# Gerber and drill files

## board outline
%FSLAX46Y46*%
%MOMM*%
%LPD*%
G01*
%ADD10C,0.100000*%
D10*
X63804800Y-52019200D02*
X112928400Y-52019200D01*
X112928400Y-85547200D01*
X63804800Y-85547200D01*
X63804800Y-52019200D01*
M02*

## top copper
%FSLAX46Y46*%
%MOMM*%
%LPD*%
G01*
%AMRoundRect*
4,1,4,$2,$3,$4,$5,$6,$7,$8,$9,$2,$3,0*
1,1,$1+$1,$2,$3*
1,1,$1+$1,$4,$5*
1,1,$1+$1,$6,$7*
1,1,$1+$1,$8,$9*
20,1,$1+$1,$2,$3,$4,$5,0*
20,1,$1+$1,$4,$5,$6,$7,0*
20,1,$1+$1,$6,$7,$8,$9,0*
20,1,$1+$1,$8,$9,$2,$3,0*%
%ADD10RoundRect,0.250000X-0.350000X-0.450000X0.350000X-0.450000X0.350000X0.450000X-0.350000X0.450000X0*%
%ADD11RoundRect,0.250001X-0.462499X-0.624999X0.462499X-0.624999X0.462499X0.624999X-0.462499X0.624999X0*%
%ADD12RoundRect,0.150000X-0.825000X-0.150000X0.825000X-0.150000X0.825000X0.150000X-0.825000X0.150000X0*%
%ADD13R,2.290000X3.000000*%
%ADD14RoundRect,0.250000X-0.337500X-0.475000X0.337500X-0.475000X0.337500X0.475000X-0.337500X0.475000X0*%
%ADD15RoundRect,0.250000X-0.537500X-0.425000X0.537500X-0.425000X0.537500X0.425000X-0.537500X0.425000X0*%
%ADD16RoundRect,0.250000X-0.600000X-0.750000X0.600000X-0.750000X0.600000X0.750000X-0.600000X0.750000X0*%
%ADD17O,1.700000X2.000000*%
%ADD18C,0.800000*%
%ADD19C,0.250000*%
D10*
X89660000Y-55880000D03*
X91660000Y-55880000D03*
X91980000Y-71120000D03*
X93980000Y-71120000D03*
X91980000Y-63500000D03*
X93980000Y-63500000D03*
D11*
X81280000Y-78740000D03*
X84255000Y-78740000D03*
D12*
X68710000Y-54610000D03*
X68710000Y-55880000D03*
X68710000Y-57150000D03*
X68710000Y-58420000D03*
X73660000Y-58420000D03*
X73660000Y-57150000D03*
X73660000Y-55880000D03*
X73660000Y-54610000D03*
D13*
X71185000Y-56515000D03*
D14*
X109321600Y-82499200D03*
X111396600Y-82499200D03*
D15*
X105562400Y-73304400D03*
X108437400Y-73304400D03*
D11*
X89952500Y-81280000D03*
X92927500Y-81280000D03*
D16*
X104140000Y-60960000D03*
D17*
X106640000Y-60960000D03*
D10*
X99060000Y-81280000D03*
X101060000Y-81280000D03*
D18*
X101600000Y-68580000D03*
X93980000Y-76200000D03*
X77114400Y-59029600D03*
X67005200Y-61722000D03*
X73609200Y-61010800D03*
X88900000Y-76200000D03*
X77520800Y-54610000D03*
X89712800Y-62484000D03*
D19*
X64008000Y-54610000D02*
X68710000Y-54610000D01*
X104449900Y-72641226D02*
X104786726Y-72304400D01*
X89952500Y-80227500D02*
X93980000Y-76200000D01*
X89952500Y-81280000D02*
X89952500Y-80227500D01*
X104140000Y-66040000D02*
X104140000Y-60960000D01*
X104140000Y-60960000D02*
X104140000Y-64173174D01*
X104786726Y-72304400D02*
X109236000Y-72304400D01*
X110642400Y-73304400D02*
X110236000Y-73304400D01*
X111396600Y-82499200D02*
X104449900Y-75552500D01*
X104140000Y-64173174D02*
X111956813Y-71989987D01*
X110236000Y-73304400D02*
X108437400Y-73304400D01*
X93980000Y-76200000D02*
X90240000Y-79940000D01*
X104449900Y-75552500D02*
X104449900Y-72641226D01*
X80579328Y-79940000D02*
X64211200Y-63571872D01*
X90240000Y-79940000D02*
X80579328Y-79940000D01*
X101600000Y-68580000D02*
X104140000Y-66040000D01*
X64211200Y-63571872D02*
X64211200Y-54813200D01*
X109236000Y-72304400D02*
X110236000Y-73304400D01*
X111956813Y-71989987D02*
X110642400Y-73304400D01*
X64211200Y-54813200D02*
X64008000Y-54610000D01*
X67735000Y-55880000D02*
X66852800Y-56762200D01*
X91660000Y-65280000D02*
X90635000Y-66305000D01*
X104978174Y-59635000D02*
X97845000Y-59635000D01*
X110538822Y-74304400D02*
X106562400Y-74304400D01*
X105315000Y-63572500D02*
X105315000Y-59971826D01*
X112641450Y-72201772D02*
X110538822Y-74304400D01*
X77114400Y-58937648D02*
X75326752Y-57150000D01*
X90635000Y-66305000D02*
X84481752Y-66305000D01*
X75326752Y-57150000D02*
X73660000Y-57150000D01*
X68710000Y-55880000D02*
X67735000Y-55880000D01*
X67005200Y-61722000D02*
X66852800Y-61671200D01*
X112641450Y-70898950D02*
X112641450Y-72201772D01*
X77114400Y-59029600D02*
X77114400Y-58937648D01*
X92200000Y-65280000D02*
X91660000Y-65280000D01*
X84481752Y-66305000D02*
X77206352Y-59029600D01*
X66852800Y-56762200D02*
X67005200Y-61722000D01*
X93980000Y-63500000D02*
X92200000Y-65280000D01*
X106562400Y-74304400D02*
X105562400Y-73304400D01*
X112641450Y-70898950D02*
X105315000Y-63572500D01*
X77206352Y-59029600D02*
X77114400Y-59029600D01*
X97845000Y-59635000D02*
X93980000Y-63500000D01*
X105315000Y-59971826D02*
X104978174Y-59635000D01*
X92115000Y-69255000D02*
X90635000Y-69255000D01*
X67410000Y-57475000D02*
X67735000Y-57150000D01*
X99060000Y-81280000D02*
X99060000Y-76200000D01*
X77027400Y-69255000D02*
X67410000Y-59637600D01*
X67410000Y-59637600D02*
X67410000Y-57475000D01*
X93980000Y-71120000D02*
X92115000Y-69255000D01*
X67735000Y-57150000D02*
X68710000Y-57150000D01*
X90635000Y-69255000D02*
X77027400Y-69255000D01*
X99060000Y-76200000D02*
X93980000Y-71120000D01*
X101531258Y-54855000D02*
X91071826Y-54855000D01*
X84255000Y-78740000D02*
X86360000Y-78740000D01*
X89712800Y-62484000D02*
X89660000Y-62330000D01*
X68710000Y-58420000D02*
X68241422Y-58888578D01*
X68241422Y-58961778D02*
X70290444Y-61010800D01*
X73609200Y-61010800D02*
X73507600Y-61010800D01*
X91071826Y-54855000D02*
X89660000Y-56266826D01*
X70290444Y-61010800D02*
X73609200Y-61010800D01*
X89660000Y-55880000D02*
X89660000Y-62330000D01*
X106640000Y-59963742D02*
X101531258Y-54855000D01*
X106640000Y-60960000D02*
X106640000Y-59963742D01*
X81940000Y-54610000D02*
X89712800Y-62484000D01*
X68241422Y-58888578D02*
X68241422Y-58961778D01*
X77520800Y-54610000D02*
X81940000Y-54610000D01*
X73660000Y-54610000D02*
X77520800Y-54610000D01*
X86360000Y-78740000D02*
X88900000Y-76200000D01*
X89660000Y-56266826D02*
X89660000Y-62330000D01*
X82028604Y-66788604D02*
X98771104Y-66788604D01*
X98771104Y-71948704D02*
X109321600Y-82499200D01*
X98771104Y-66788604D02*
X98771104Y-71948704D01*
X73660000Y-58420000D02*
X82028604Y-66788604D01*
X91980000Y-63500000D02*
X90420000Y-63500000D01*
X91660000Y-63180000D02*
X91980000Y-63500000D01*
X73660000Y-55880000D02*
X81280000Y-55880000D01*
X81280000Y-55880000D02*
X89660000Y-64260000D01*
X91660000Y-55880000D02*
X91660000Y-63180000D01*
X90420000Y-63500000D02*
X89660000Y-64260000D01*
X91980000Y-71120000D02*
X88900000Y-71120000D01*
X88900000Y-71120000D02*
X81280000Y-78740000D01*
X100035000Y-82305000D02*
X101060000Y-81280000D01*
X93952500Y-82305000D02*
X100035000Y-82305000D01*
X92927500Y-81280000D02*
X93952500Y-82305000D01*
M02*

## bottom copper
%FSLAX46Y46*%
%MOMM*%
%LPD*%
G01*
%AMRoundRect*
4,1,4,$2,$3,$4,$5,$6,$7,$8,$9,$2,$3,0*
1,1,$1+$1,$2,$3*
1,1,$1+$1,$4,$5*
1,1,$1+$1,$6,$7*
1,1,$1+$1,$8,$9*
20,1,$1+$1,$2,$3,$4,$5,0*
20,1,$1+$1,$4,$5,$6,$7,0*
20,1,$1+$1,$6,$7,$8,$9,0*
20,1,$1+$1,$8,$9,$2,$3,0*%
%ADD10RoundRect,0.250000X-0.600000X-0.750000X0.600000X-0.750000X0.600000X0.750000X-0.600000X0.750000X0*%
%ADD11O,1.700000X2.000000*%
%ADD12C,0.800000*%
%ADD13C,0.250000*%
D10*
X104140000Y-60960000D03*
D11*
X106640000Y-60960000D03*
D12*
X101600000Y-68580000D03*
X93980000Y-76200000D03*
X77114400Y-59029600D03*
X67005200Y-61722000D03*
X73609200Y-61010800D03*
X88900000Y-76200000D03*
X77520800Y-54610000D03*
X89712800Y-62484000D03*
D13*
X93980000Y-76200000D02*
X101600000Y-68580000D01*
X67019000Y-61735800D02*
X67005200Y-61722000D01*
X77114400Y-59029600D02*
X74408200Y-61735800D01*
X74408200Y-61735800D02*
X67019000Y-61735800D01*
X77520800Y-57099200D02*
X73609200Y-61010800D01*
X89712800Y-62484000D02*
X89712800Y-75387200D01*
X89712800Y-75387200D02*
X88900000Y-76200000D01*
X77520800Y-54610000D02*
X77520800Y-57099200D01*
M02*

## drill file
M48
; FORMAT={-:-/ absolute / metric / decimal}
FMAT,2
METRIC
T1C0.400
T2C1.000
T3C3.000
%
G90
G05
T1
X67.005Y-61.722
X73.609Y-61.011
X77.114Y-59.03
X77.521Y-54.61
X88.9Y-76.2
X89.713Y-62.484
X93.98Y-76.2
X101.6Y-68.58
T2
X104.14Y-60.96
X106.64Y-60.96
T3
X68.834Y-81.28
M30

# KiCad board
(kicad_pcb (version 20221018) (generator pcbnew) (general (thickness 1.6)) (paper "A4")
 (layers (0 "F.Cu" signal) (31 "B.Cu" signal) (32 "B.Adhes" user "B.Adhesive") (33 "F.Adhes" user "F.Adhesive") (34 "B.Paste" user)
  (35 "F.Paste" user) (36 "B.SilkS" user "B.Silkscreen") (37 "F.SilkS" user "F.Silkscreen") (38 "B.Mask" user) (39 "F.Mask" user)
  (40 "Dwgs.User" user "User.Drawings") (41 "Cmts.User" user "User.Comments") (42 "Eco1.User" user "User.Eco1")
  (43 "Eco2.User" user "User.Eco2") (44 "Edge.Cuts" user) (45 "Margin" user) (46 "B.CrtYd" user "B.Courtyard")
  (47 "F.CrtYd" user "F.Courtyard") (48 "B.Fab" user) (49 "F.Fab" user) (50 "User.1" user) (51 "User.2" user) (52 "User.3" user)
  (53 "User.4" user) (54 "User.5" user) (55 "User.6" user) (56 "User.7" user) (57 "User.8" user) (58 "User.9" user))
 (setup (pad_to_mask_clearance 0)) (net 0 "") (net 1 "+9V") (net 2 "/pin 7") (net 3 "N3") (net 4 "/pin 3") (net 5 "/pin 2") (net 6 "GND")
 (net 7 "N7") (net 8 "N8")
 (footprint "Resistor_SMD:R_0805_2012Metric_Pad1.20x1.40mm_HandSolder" (layer "F.Cu") (at 90.66 55.88)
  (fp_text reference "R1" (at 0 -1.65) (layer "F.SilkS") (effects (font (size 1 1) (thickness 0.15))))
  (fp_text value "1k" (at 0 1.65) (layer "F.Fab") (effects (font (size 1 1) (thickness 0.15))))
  (pad "1" smd roundrect (at -1 0) (size 1.2 1.4) (layers "F.Cu" "F.Paste" "F.Mask") (roundrect_rratio 0.2083333333) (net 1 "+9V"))
  (pad "2" smd roundrect (at 1 0) (size 1.2 1.4) (layers "F.Cu" "F.Paste" "F.Mask") (roundrect_rratio 0.2083333333) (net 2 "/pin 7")))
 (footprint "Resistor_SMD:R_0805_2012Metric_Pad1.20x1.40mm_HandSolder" (layer "F.Cu") (at 92.98 71.12)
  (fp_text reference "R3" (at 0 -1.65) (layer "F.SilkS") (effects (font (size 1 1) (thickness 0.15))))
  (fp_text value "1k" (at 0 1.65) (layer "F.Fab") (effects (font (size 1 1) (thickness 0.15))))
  (pad "1" smd roundrect (at -1 0) (size 1.2 1.4) (layers "F.Cu" "F.Paste" "F.Mask") (roundrect_rratio 0.2083333333) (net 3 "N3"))
  (pad "2" smd roundrect (at 1 0) (size 1.2 1.4) (layers "F.Cu" "F.Paste" "F.Mask") (roundrect_rratio 0.2083333333) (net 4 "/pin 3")))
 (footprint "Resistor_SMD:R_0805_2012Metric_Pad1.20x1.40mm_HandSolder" (layer "F.Cu") (at 92.98 63.5)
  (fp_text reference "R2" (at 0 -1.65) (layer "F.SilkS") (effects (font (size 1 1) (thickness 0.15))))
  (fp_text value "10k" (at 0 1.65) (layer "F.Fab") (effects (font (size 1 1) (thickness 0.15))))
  (pad "1" smd roundrect (at -1 0) (size 1.2 1.4) (layers "F.Cu" "F.Paste" "F.Mask") (roundrect_rratio 0.2083333333) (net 2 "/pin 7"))
  (pad "2" smd roundrect (at 1 0) (size 1.2 1.4) (layers "F.Cu" "F.Paste" "F.Mask") (roundrect_rratio 0.2083333333) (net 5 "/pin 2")))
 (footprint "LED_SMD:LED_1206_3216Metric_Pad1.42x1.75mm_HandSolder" (layer "F.Cu") (at 82.7675 78.74)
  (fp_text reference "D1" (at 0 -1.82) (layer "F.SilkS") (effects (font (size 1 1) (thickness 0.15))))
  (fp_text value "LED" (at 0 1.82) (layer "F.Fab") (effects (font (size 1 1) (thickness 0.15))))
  (pad "1" smd roundrect (at -1.4875 0) (size 1.425 1.75) (layers "F.Cu" "F.Paste" "F.Mask") (roundrect_rratio 0.1754392982) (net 3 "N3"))
  (pad "2" smd roundrect (at 1.4875 0) (size 1.425 1.75) (layers "F.Cu" "F.Paste" "F.Mask") (roundrect_rratio 0.1754392982) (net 1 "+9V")))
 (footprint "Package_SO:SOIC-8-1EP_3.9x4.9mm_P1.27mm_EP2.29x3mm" (layer "F.Cu") (at 71.185 56.515)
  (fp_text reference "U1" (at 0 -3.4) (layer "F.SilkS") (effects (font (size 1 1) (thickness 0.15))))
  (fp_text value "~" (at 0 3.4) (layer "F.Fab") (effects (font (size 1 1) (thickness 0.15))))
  (pad "" smd roundrect (at -0.57 -0.75) (size 0.92 1.21) (layers "F.Paste") (roundrect_rratio 0.25))
  (pad "" smd roundrect (at -0.57 0.75) (size 0.92 1.21) (layers "F.Paste") (roundrect_rratio 0.25))
  (pad "" smd roundrect (at 0.57 -0.75) (size 0.92 1.21) (layers "F.Paste") (roundrect_rratio 0.25))
  (pad "" smd roundrect (at 0.57 0.75) (size 0.92 1.21) (layers "F.Paste") (roundrect_rratio 0.25))
  (pad "1" smd roundrect (at -2.475 -1.905) (size 1.95 0.6) (layers "F.Cu" "F.Paste" "F.Mask") (roundrect_rratio 0.25) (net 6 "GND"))
  (pad "2" smd roundrect (at -2.475 -0.635) (size 1.95 0.6) (layers "F.Cu" "F.Paste" "F.Mask") (roundrect_rratio 0.25) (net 5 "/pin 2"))
  (pad "3" smd roundrect (at -2.475 0.635) (size 1.95 0.6) (layers "F.Cu" "F.Paste" "F.Mask") (roundrect_rratio 0.25) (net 4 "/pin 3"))
  (pad "4" smd roundrect (at -2.475 1.905) (size 1.95 0.6) (layers "F.Cu" "F.Paste" "F.Mask") (roundrect_rratio 0.25) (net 1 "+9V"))
  (pad "5" smd roundrect (at 2.475 1.905) (size 1.95 0.6) (layers "F.Cu" "F.Paste" "F.Mask") (roundrect_rratio 0.25) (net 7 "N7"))
  (pad "6" smd roundrect (at 2.475 0.635) (size 1.95 0.6) (layers "F.Cu" "F.Paste" "F.Mask") (roundrect_rratio 0.25) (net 5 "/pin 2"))
  (pad "7" smd roundrect (at 2.475 -0.635) (size 1.95 0.6) (layers "F.Cu" "F.Paste" "F.Mask") (roundrect_rratio 0.25) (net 2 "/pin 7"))
  (pad "8" smd roundrect (at 2.475 -1.905) (size 1.95 0.6) (layers "F.Cu" "F.Paste" "F.Mask") (roundrect_rratio 0.25) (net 1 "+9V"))
  (pad "9" smd rect (at 0 0) (size 2.29 3) (layers "F.Cu" "F.Mask")))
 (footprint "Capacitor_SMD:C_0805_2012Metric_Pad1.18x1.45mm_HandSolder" (layer "F.Cu") (at 110.3591 82.4992)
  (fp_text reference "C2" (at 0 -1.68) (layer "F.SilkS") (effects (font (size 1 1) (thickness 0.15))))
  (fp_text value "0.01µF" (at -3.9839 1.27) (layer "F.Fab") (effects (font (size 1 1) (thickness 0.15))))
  (pad "1" smd roundrect (at -1.0375 0) (size 1.175 1.45) (layers "F.Cu" "F.Paste" "F.Mask") (roundrect_rratio 0.2127659574) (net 7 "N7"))
  (pad "2" smd roundrect (at 1.0375 0) (size 1.175 1.45) (layers "F.Cu" "F.Paste" "F.Mask") (roundrect_rratio 0.2127659574) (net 6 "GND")))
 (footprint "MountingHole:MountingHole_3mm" (layer "F.Cu") (at 68.834 81.28)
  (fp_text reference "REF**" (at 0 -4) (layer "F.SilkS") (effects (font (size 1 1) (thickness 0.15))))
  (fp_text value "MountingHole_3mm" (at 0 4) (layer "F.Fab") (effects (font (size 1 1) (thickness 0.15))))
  (pad "" np_thru_hole circle (at 0 0) (size 3 3) (drill 3) (layers "*.Cu" "*.Mask")))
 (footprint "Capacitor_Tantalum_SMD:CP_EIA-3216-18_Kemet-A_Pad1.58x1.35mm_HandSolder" (layer "F.Cu") (at 106.9999 73.3044)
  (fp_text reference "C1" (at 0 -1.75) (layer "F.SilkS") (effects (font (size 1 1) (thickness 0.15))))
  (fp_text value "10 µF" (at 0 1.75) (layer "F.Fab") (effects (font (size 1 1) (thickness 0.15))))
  (pad "1" smd roundrect (at -1.4375 0) (size 1.575 1.35) (layers "F.Cu" "F.Paste" "F.Mask") (roundrect_rratio 0.1851851852)
   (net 5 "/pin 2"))
  (pad "2" smd roundrect (at 1.4375 0) (size 1.575 1.35) (layers "F.Cu" "F.Paste" "F.Mask") (roundrect_rratio 0.1851851852) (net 6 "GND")))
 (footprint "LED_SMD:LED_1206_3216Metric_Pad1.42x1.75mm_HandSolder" (layer "F.Cu") (at 91.44 81.28)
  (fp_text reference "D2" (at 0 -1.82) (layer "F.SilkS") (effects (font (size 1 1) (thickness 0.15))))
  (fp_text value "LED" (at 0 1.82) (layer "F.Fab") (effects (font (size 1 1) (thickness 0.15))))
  (pad "1" smd roundrect (at -1.4875 0) (size 1.425 1.75) (layers "F.Cu" "F.Paste" "F.Mask") (roundrect_rratio 0.1754392982) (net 6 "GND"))
  (pad "2" smd roundrect (at 1.4875 0) (size 1.425 1.75) (layers "F.Cu" "F.Paste" "F.Mask") (roundrect_rratio 0.1754392982) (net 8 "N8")))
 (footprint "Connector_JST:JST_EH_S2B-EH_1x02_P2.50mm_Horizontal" (layer "F.Cu") (at 104.14 60.96)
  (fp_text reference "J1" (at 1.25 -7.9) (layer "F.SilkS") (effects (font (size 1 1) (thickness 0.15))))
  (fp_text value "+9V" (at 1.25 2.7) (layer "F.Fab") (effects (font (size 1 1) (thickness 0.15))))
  (pad "1" thru_hole roundrect (at 0 0) (size 1.7 2) (drill 1) (layers "*.Cu" "*.Mask") (roundrect_rratio 0.1470588235) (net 6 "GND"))
  (pad "2" thru_hole oval (at 2.5 0) (size 1.7 2) (drill 1) (layers "*.Cu" "*.Mask") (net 1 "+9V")))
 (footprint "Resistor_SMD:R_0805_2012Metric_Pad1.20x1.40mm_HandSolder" (layer "F.Cu") (at 100.06 81.28)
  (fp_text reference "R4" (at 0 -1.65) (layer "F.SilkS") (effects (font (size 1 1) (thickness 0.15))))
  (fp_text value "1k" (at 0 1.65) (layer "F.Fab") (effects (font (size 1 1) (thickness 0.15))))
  (pad "1" smd roundrect (at -1 0) (size 1.2 1.4) (layers "F.Cu" "F.Paste" "F.Mask") (roundrect_rratio 0.2083333333) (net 4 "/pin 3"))
  (pad "2" smd roundrect (at 1 0) (size 1.2 1.4) (layers "F.Cu" "F.Paste" "F.Mask") (roundrect_rratio 0.2083333333) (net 8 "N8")))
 (gr_rect (start 63.8048 52.0192) (end 112.9284 85.5472) (stroke (width 0.1) (type default)) (fill none) (layer "Edge.Cuts"))
 (segment (start 64.008 54.61) (end 68.71 54.61) (width 0.25) (layer "F.Cu") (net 6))
 (segment (start 104.4499 72.641226) (end 104.786726 72.3044) (width 0.25) (layer "F.Cu") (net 6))
 (segment (start 89.9525 80.2275) (end 93.98 76.2) (width 0.25) (layer "F.Cu") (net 6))
 (segment (start 89.9525 81.28) (end 89.9525 80.2275) (width 0.25) (layer "F.Cu") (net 6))
 (segment (start 104.14 66.04) (end 104.14 60.96) (width 0.25) (layer "F.Cu") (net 6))
 (segment (start 104.14 60.96) (end 104.14 64.173174) (width 0.25) (layer "F.Cu") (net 6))
 (segment (start 104.786726 72.3044) (end 109.236 72.3044) (width 0.25) (layer "F.Cu") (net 6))
 (segment (start 110.6424 73.3044) (end 110.236 73.3044) (width 0.25) (layer "F.Cu") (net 6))
 (segment (start 111.3966 82.4992) (end 104.4499 75.5525) (width 0.25) (layer "F.Cu") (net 6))
 (segment (start 104.14 64.173174) (end 111.956813 71.989987) (width 0.25) (layer "F.Cu") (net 6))
 (segment (start 110.236 73.3044) (end 108.4374 73.3044) (width 0.25) (layer "F.Cu") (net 6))
 (segment (start 93.98 76.2) (end 90.24 79.94) (width 0.25) (layer "F.Cu") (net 6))
 (segment (start 104.4499 75.5525) (end 104.4499 72.641226) (width 0.25) (layer "F.Cu") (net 6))
 (segment (start 80.579328 79.94) (end 64.2112 63.571872) (width 0.25) (layer "F.Cu") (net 6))
 (segment (start 90.24 79.94) (end 80.579328 79.94) (width 0.25) (layer "F.Cu") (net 6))
 (segment (start 101.6 68.58) (end 104.14 66.04) (width 0.25) (layer "F.Cu") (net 6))
 (segment (start 64.2112 63.571872) (end 64.2112 54.8132) (width 0.25) (layer "F.Cu") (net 6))
 (segment (start 109.236 72.3044) (end 110.236 73.3044) (width 0.25) (layer "F.Cu") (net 6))
 (segment (start 111.956813 71.989987) (end 110.6424 73.3044) (width 0.25) (layer "F.Cu") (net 6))
 (segment (start 64.2112 54.8132) (end 64.008 54.61) (width 0.25) (layer "F.Cu") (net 6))
 (via (at 101.6 68.58) (size 0.8) (drill 0.4) (layers "F.Cu" "B.Cu") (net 6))
 (via (at 93.98 76.2) (size 0.8) (drill 0.4) (layers "F.Cu" "B.Cu") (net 6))
 (segment (start 93.98 76.2) (end 101.6 68.58) (width 0.25) (layer "B.Cu") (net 6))
 (segment (start 67.735 55.88) (end 66.8528 56.7622) (width 0.25) (layer "F.Cu") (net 5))
 (segment (start 91.66 65.28) (end 90.635 66.305) (width 0.25) (layer "F.Cu") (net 5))
 (segment (start 104.978174 59.635) (end 97.845 59.635) (width 0.25) (layer "F.Cu") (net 5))
 (segment (start 110.538822 74.3044) (end 106.5624 74.3044) (width 0.25) (layer "F.Cu") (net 5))
 (segment (start 105.315 63.5725) (end 105.315 59.971826) (width 0.25) (layer "F.Cu") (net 5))
 (segment (start 112.64145 72.201772) (end 110.538822 74.3044) (width 0.25) (layer "F.Cu") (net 5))
 (segment (start 77.1144 58.937648) (end 75.326752 57.15) (width 0.25) (layer "F.Cu") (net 5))
 (segment (start 90.635 66.305) (end 84.481752 66.305) (width 0.25) (layer "F.Cu") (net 5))
 (segment (start 75.326752 57.15) (end 73.66 57.15) (width 0.25) (layer "F.Cu") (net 5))
 (segment (start 68.71 55.88) (end 67.735 55.88) (width 0.25) (layer "F.Cu") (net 5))
 (segment (start 67.0052 61.722) (end 66.8528 61.6712) (width 0.25) (layer "F.Cu") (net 5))
 (segment (start 112.64145 70.89895) (end 112.64145 72.201772) (width 0.25) (layer "F.Cu") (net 5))
 (segment (start 77.1144 59.0296) (end 77.1144 58.937648) (width 0.25) (layer "F.Cu") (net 5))
 (segment (start 92.2 65.28) (end 91.66 65.28) (width 0.25) (layer "F.Cu") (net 5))
 (segment (start 84.481752 66.305) (end 77.206352 59.0296) (width 0.25) (layer "F.Cu") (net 5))
 (segment (start 66.8528 56.7622) (end 67.0052 61.722) (width 0.25) (layer "F.Cu") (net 5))
 (segment (start 93.98 63.5) (end 92.2 65.28) (width 0.25) (layer "F.Cu") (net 5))
 (segment (start 106.5624 74.3044) (end 105.5624 73.3044) (width 0.25) (layer "F.Cu") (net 5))
 (segment (start 112.64145 70.89895) (end 105.315 63.5725) (width 0.25) (layer "F.Cu") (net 5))
 (segment (start 77.206352 59.0296) (end 77.1144 59.0296) (width 0.25) (layer "F.Cu") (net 5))
 (segment (start 97.845 59.635) (end 93.98 63.5) (width 0.25) (layer "F.Cu") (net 5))
 (segment (start 105.315 59.971826) (end 104.978174 59.635) (width 0.25) (layer "F.Cu") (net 5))
 (via (at 77.1144 59.0296) (size 0.8) (drill 0.4) (layers "F.Cu" "B.Cu") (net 5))
 (via (at 67.0052 61.722) (size 0.8) (drill 0.4) (layers "F.Cu" "B.Cu") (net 5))
 (segment (start 67.019 61.7358) (end 67.0052 61.722) (width 0.25) (layer "B.Cu") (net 5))
 (segment (start 77.1144 59.0296) (end 74.4082 61.7358) (width 0.25) (layer "B.Cu") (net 5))
 (segment (start 74.4082 61.7358) (end 67.019 61.7358) (width 0.25) (layer "B.Cu") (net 5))
 (segment (start 92.115 69.255) (end 90.635 69.255) (width 0.25) (layer "F.Cu") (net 4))
 (segment (start 67.41 57.475) (end 67.735 57.15) (width 0.25) (layer "F.Cu") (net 4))
 (segment (start 99.06 81.28) (end 99.06 76.2) (width 0.25) (layer "F.Cu") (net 4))
 (segment (start 77.0274 69.255) (end 67.41 59.6376) (width 0.25) (layer "F.Cu") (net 4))
 (segment (start 67.41 59.6376) (end 67.41 57.475) (width 0.25) (layer "F.Cu") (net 4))
 (segment (start 93.98 71.12) (end 92.115 69.255) (width 0.25) (layer "F.Cu") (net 4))
 (segment (start 67.735 57.15) (end 68.71 57.15) (width 0.25) (layer "F.Cu") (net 4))
 (segment (start 90.635 69.255) (end 77.0274 69.255) (width 0.25) (layer "F.Cu") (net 4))
 (segment (start 99.06 76.2) (end 93.98 71.12) (width 0.25) (layer "F.Cu") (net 4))
 (segment (start 101.531258 54.855) (end 91.071826 54.855) (width 0.25) (layer "F.Cu") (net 1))
 (segment (start 84.255 78.74) (end 86.36 78.74) (width 0.25) (layer "F.Cu") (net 1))
 (segment (start 89.7128 62.484) (end 89.66 62.33) (width 0.25) (layer "F.Cu") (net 1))
 (segment (start 68.71 58.42) (end 68.241422 58.888578) (width 0.25) (layer "F.Cu") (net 1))
 (segment (start 68.241422 58.961778) (end 70.290444 61.0108) (width 0.25) (layer "F.Cu") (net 1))
 (segment (start 73.6092 61.0108) (end 73.5076 61.0108) (width 0.25) (layer "F.Cu") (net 1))
 (segment (start 91.071826 54.855) (end 89.66 56.266826) (width 0.25) (layer "F.Cu") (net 1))
 (segment (start 70.290444 61.0108) (end 73.6092 61.0108) (width 0.25) (layer "F.Cu") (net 1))
 (segment (start 89.66 55.88) (end 89.66 62.33) (width 0.25) (layer "F.Cu") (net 1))
 (segment (start 106.64 59.963742) (end 101.531258 54.855) (width 0.25) (layer "F.Cu") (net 1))
 (segment (start 106.64 60.96) (end 106.64 59.963742) (width 0.25) (layer "F.Cu") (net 1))
 (segment (start 81.94 54.61) (end 89.7128 62.484) (width 0.25) (layer "F.Cu") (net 1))
 (segment (start 68.241422 58.888578) (end 68.241422 58.961778) (width 0.25) (layer "F.Cu") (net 1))
 (segment (start 77.5208 54.61) (end 81.94 54.61) (width 0.25) (layer "F.Cu") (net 1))
 (segment (start 73.66 54.61) (end 77.5208 54.61) (width 0.25) (layer "F.Cu") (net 1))
 (segment (start 86.36 78.74) (end 88.9 76.2) (width 0.25) (layer "F.Cu") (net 1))
 (segment (start 89.66 56.266826) (end 89.66 62.33) (width 0.25) (layer "F.Cu") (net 1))
 (via (at 73.6092 61.0108) (size 0.8) (drill 0.4) (layers "F.Cu" "B.Cu") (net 1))
 (via (at 88.9 76.2) (size 0.8) (drill 0.4) (layers "F.Cu" "B.Cu") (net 1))
 (via (at 77.5208 54.61) (size 0.8) (drill 0.4) (layers "F.Cu" "B.Cu") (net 1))
 (via (at 89.7128 62.484) (size 0.8) (drill 0.4) (layers "F.Cu" "B.Cu") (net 1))
 (segment (start 77.5208 57.0992) (end 73.6092 61.0108) (width 0.25) (layer "B.Cu") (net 1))
 (segment (start 89.7128 62.484) (end 89.7128 75.3872) (width 0.25) (layer "B.Cu") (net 1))
 (segment (start 89.7128 75.3872) (end 88.9 76.2) (width 0.25) (layer "B.Cu") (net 1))
 (segment (start 77.5208 54.61) (end 77.5208 57.0992) (width 0.25) (layer "B.Cu") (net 1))
 (segment (start 82.028604 66.788604) (end 98.771104 66.788604) (width 0.25) (layer "F.Cu") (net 7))
 (segment (start 98.771104 71.948704) (end 109.3216 82.4992) (width 0.25) (layer "F.Cu") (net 7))
 (segment (start 98.771104 66.788604) (end 98.771104 71.948704) (width 0.25) (layer "F.Cu") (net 7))
 (segment (start 73.66 58.42) (end 82.028604 66.788604) (width 0.25) (layer "F.Cu") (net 7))
 (segment (start 91.98 63.5) (end 90.42 63.5) (width 0.25) (layer "F.Cu") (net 2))
 (segment (start 91.66 63.18) (end 91.98 63.5) (width 0.25) (layer "F.Cu") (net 2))
 (segment (start 73.66 55.88) (end 81.28 55.88) (width 0.25) (layer "F.Cu") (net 2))
 (segment (start 81.28 55.88) (end 89.66 64.26) (width 0.25) (layer "F.Cu") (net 2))
 (segment (start 91.66 55.88) (end 91.66 63.18) (width 0.25) (layer "F.Cu") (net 2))
 (segment (start 90.42 63.5) (end 89.66 64.26) (width 0.25) (layer "F.Cu") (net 2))
 (segment (start 91.98 71.12) (end 88.9 71.12) (width 0.25) (layer "F.Cu") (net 3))
 (segment (start 88.9 71.12) (end 81.28 78.74) (width 0.25) (layer "F.Cu") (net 3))
 (segment (start 100.035 82.305) (end 101.06 81.28) (width 0.25) (layer "F.Cu") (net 8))
 (segment (start 93.9525 82.305) (end 100.035 82.305) (width 0.25) (layer "F.Cu") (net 8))
 (segment (start 92.9275 81.28) (end 93.9525 82.305) (width 0.25) (layer "F.Cu") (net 8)))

